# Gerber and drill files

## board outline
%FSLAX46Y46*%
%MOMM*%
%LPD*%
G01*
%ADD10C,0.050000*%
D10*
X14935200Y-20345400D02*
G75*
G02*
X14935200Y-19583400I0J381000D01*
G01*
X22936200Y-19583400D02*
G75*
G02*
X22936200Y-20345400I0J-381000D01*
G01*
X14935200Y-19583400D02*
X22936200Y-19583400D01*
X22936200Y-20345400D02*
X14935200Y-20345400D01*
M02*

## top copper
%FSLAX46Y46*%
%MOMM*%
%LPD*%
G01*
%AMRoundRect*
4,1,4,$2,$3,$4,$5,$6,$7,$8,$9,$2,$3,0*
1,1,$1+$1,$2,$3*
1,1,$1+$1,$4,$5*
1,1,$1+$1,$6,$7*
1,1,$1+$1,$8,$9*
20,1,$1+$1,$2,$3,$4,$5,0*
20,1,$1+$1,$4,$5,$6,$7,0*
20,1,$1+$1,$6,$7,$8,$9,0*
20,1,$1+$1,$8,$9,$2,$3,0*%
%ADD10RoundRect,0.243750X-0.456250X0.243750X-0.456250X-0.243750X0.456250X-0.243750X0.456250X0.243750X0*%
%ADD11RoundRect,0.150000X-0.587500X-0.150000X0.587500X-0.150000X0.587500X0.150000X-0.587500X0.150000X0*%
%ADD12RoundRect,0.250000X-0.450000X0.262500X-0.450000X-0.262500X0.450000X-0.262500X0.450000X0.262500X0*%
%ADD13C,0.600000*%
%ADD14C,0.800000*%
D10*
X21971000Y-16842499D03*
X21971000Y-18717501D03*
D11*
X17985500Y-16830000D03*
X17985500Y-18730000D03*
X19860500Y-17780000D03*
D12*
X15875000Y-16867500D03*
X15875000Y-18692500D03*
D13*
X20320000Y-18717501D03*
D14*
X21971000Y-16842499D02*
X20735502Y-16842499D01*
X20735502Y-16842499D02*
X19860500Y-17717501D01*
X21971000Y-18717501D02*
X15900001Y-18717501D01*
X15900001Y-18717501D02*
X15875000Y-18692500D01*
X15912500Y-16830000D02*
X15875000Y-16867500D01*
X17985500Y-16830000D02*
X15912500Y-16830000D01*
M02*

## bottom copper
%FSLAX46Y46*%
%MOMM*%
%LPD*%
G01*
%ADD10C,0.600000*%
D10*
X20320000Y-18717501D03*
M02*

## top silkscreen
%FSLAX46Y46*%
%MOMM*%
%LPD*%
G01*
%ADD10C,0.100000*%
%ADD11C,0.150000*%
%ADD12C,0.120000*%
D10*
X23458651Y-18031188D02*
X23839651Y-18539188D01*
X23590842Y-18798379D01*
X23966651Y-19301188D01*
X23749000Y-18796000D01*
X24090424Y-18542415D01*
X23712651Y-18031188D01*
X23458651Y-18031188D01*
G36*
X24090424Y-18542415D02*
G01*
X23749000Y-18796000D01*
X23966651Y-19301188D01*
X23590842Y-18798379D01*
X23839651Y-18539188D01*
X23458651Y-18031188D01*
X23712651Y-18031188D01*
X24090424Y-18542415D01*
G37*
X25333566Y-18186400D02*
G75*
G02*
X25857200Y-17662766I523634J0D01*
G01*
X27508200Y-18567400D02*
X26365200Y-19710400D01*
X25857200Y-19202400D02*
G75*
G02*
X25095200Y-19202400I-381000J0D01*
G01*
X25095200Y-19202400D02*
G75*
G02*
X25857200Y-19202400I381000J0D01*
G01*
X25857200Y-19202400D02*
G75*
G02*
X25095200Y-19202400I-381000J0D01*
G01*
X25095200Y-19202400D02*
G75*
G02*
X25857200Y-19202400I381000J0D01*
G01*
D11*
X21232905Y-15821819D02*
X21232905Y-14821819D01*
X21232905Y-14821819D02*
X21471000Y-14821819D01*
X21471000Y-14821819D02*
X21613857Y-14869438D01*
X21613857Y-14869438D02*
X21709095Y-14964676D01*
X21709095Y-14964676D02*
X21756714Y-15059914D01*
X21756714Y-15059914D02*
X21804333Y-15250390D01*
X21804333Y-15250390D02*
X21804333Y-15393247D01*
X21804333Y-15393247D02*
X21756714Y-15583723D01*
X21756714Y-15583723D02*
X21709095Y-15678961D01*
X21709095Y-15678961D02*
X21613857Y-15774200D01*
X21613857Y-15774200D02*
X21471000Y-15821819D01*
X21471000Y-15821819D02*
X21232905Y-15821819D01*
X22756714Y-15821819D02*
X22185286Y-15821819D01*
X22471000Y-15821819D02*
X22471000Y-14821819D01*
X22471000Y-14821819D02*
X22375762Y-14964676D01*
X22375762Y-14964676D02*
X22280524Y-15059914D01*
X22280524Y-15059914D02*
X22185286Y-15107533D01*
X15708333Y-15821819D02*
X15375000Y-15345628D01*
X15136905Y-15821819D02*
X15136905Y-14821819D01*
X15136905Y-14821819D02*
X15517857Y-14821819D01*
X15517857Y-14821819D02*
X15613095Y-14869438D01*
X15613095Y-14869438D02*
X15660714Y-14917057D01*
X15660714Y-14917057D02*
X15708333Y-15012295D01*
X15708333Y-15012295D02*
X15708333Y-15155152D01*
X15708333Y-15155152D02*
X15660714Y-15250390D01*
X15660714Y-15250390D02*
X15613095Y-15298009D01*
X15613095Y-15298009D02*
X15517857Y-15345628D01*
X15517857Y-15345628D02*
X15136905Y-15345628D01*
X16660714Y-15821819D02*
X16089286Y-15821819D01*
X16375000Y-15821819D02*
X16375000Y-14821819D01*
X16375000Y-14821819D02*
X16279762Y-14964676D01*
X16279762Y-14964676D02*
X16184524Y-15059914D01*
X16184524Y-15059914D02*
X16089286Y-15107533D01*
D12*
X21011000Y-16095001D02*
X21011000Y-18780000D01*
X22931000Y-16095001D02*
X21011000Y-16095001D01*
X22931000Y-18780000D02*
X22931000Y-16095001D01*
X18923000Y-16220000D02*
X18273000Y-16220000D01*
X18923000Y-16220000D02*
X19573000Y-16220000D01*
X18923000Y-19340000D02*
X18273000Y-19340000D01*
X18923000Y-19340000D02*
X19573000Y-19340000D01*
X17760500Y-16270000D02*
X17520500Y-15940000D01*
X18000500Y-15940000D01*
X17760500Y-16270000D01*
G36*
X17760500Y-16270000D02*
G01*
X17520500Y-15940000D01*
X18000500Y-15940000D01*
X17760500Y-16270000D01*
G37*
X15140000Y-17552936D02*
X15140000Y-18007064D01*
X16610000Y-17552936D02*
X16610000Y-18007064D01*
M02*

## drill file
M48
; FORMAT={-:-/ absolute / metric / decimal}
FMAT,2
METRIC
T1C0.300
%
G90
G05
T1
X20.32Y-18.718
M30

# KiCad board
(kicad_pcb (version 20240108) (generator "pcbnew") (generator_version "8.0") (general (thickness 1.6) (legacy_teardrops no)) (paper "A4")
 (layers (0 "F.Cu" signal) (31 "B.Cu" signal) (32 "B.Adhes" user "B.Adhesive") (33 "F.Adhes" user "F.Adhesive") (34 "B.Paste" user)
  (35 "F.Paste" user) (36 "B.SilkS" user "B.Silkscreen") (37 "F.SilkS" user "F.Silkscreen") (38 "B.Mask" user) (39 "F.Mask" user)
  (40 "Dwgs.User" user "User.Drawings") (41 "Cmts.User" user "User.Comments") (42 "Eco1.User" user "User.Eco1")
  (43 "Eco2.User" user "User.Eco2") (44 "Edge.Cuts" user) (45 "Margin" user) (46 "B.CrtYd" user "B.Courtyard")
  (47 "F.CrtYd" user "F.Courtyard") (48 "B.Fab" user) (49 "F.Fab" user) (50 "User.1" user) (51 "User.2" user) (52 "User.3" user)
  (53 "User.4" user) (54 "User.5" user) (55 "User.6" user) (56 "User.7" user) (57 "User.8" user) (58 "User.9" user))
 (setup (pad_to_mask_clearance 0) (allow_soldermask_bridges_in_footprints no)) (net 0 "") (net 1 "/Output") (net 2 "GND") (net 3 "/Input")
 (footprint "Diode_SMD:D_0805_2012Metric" (layer "F.Cu") (at 21.971 17.78 -90)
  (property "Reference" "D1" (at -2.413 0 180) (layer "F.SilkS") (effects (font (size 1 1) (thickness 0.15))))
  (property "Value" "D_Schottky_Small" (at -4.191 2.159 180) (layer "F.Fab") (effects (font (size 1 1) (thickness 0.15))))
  (fp_line (start -1.684999 0.96) (end 1 0.96) (stroke (width 0.12) (type solid)) (layer "F.SilkS"))
  (fp_line (start -1.684999 -0.96) (end -1.684999 0.96) (stroke (width 0.12) (type solid)) (layer "F.SilkS"))
  (fp_line (start 1 -0.96) (end -1.684999 -0.96) (stroke (width 0.12) (type solid)) (layer "F.SilkS"))
  (pad "1" smd roundrect (at -0.937501 0 270) (size 0.975 1.4) (layers "F.Cu" "F.Paste" "F.Mask") (roundrect_rratio 0.25) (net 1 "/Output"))
  (pad "2" smd roundrect (at 0.937501 0 270) (size 0.975 1.4) (layers "F.Cu" "F.Paste" "F.Mask") (roundrect_rratio 0.25) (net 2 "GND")))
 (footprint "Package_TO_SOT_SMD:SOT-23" (layer "F.Cu") (at 18.923 17.78)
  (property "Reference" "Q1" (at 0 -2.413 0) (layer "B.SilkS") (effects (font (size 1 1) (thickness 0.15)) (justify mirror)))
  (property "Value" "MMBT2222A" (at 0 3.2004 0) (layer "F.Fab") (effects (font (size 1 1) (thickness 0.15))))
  (fp_line (start 0 -1.56) (end -0.65 -1.56) (stroke (width 0.12) (type solid)) (layer "F.SilkS"))
  (fp_line (start 0 -1.56) (end 0.65 -1.56) (stroke (width 0.12) (type solid)) (layer "F.SilkS"))
  (fp_line (start 0 1.56) (end -0.65 1.56) (stroke (width 0.12) (type solid)) (layer "F.SilkS"))
  (fp_line (start 0 1.56) (end 0.65 1.56) (stroke (width 0.12) (type solid)) (layer "F.SilkS"))
  (fp_poly
   (pts (xy -1.1625 -1.51) (xy -1.4025 -1.84) (xy -0.9225 -1.84) (xy -1.1625 -1.51)) (stroke (width 0.12) (type solid)) (fill solid)
   (layer "F.SilkS"))
  (pad "1" smd roundrect (at -0.9375 -0.95) (size 1.475 0.6) (layers "F.Cu" "F.Paste" "F.Mask") (roundrect_rratio 0.25) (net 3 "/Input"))
  (pad "2" smd roundrect (at -0.9375 0.95) (size 1.475 0.6) (layers "F.Cu" "F.Paste" "F.Mask") (roundrect_rratio 0.25) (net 2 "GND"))
  (pad "3" smd roundrect (at 0.9375 0) (size 1.475 0.6) (layers "F.Cu" "F.Paste" "F.Mask") (roundrect_rratio 0.25) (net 1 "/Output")))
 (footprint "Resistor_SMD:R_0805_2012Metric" (layer "F.Cu") (at 15.875 17.78 -90)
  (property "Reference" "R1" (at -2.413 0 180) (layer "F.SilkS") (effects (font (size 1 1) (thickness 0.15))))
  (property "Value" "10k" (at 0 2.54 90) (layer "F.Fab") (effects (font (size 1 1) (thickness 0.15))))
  (fp_line (start -0.227064 0.735) (end 0.227064 0.735) (stroke (width 0.12) (type solid)) (layer "F.SilkS"))
  (fp_line (start -0.227064 -0.735) (end 0.227064 -0.735) (stroke (width 0.12) (type solid)) (layer "F.SilkS"))
  (pad "1" smd roundrect (at -0.9125 0 270) (size 1.025 1.4) (layers "F.Cu" "F.Paste" "F.Mask") (roundrect_rratio 0.243902) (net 3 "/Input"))
  (pad "2" smd roundrect (at 0.9125 0 270) (size 1.025 1.4) (layers "F.Cu" "F.Paste" "F.Mask") (roundrect_rratio 0.243902) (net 2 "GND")))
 (gr_poly
  (pts (xy 23.458651 18.031188) (xy 23.839651 18.539188) (xy 23.590842 18.798379) (xy 23.966651 19.301188) (xy 23.749 18.796)
   (xy 24.090424 18.542415) (xy 23.712651 18.031188))
  (stroke (width 0.1) (type solid)) (fill solid) (layer "F.SilkS"))
 (gr_arc (start 25.333566 18.1864) (mid 25.486935 17.816135) (end 25.8572 17.662766) (stroke (width 0.1) (type default)) (layer "F.SilkS"))
 (gr_line (start 27.5082 18.5674) (end 26.3652 19.7104) (stroke (width 0.1) (type default)) (layer "F.SilkS"))
 (gr_circle (center 25.4762 19.2024) (end 25.4762 18.8214) (stroke (width 0.1) (type default)) (fill none) (layer "F.SilkS"))
 (gr_circle (center 25.4762 19.2024) (end 25.4762 18.8214) (stroke (width 0.1) (type default)) (fill none) (layer "F.SilkS"))
 (gr_arc (start 14.9352 20.3454) (mid 14.5542 19.9644) (end 14.9352 19.5834) (stroke (width 0.05) (type default)) (layer "Edge.Cuts"))
 (gr_arc (start 22.9362 19.5834) (mid 23.3172 19.9644) (end 22.9362 20.3454) (stroke (width 0.05) (type default)) (layer "Edge.Cuts"))
 (gr_line (start 14.9352 19.5834) (end 22.9362 19.5834) (stroke (width 0.05) (type default)) (layer "Edge.Cuts"))
 (gr_line (start 22.9362 20.3454) (end 14.9352 20.3454) (stroke (width 0.05) (type default)) (layer "Edge.Cuts"))
 (segment (start 21.971 16.842499) (end 20.735502 16.842499) (width 0.8) (layer "F.Cu") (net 1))
 (segment (start 20.735502 16.842499) (end 19.8605 17.717501) (width 0.8) (layer "F.Cu") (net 1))
 (segment (start 21.971 18.717501) (end 15.900001 18.717501) (width 0.8) (layer "F.Cu") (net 2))
 (segment (start 15.900001 18.717501) (end 15.875 18.6925) (width 0.8) (layer "F.Cu") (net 2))
 (via (at 20.32 18.717501) (size 0.6) (drill 0.3) (layers "F.Cu" "B.Cu") (free yes) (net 2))
 (segment (start 15.9125 16.83) (end 15.875 16.8675) (width 0.8) (layer "F.Cu") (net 3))
 (segment (start 17.9855 16.83) (end 15.9125 16.83) (width 0.8) (layer "F.Cu") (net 3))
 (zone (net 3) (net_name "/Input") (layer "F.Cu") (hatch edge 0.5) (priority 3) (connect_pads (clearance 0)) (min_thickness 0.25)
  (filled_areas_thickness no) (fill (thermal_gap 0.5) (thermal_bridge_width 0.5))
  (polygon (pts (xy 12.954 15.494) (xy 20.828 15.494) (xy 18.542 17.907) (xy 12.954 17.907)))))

